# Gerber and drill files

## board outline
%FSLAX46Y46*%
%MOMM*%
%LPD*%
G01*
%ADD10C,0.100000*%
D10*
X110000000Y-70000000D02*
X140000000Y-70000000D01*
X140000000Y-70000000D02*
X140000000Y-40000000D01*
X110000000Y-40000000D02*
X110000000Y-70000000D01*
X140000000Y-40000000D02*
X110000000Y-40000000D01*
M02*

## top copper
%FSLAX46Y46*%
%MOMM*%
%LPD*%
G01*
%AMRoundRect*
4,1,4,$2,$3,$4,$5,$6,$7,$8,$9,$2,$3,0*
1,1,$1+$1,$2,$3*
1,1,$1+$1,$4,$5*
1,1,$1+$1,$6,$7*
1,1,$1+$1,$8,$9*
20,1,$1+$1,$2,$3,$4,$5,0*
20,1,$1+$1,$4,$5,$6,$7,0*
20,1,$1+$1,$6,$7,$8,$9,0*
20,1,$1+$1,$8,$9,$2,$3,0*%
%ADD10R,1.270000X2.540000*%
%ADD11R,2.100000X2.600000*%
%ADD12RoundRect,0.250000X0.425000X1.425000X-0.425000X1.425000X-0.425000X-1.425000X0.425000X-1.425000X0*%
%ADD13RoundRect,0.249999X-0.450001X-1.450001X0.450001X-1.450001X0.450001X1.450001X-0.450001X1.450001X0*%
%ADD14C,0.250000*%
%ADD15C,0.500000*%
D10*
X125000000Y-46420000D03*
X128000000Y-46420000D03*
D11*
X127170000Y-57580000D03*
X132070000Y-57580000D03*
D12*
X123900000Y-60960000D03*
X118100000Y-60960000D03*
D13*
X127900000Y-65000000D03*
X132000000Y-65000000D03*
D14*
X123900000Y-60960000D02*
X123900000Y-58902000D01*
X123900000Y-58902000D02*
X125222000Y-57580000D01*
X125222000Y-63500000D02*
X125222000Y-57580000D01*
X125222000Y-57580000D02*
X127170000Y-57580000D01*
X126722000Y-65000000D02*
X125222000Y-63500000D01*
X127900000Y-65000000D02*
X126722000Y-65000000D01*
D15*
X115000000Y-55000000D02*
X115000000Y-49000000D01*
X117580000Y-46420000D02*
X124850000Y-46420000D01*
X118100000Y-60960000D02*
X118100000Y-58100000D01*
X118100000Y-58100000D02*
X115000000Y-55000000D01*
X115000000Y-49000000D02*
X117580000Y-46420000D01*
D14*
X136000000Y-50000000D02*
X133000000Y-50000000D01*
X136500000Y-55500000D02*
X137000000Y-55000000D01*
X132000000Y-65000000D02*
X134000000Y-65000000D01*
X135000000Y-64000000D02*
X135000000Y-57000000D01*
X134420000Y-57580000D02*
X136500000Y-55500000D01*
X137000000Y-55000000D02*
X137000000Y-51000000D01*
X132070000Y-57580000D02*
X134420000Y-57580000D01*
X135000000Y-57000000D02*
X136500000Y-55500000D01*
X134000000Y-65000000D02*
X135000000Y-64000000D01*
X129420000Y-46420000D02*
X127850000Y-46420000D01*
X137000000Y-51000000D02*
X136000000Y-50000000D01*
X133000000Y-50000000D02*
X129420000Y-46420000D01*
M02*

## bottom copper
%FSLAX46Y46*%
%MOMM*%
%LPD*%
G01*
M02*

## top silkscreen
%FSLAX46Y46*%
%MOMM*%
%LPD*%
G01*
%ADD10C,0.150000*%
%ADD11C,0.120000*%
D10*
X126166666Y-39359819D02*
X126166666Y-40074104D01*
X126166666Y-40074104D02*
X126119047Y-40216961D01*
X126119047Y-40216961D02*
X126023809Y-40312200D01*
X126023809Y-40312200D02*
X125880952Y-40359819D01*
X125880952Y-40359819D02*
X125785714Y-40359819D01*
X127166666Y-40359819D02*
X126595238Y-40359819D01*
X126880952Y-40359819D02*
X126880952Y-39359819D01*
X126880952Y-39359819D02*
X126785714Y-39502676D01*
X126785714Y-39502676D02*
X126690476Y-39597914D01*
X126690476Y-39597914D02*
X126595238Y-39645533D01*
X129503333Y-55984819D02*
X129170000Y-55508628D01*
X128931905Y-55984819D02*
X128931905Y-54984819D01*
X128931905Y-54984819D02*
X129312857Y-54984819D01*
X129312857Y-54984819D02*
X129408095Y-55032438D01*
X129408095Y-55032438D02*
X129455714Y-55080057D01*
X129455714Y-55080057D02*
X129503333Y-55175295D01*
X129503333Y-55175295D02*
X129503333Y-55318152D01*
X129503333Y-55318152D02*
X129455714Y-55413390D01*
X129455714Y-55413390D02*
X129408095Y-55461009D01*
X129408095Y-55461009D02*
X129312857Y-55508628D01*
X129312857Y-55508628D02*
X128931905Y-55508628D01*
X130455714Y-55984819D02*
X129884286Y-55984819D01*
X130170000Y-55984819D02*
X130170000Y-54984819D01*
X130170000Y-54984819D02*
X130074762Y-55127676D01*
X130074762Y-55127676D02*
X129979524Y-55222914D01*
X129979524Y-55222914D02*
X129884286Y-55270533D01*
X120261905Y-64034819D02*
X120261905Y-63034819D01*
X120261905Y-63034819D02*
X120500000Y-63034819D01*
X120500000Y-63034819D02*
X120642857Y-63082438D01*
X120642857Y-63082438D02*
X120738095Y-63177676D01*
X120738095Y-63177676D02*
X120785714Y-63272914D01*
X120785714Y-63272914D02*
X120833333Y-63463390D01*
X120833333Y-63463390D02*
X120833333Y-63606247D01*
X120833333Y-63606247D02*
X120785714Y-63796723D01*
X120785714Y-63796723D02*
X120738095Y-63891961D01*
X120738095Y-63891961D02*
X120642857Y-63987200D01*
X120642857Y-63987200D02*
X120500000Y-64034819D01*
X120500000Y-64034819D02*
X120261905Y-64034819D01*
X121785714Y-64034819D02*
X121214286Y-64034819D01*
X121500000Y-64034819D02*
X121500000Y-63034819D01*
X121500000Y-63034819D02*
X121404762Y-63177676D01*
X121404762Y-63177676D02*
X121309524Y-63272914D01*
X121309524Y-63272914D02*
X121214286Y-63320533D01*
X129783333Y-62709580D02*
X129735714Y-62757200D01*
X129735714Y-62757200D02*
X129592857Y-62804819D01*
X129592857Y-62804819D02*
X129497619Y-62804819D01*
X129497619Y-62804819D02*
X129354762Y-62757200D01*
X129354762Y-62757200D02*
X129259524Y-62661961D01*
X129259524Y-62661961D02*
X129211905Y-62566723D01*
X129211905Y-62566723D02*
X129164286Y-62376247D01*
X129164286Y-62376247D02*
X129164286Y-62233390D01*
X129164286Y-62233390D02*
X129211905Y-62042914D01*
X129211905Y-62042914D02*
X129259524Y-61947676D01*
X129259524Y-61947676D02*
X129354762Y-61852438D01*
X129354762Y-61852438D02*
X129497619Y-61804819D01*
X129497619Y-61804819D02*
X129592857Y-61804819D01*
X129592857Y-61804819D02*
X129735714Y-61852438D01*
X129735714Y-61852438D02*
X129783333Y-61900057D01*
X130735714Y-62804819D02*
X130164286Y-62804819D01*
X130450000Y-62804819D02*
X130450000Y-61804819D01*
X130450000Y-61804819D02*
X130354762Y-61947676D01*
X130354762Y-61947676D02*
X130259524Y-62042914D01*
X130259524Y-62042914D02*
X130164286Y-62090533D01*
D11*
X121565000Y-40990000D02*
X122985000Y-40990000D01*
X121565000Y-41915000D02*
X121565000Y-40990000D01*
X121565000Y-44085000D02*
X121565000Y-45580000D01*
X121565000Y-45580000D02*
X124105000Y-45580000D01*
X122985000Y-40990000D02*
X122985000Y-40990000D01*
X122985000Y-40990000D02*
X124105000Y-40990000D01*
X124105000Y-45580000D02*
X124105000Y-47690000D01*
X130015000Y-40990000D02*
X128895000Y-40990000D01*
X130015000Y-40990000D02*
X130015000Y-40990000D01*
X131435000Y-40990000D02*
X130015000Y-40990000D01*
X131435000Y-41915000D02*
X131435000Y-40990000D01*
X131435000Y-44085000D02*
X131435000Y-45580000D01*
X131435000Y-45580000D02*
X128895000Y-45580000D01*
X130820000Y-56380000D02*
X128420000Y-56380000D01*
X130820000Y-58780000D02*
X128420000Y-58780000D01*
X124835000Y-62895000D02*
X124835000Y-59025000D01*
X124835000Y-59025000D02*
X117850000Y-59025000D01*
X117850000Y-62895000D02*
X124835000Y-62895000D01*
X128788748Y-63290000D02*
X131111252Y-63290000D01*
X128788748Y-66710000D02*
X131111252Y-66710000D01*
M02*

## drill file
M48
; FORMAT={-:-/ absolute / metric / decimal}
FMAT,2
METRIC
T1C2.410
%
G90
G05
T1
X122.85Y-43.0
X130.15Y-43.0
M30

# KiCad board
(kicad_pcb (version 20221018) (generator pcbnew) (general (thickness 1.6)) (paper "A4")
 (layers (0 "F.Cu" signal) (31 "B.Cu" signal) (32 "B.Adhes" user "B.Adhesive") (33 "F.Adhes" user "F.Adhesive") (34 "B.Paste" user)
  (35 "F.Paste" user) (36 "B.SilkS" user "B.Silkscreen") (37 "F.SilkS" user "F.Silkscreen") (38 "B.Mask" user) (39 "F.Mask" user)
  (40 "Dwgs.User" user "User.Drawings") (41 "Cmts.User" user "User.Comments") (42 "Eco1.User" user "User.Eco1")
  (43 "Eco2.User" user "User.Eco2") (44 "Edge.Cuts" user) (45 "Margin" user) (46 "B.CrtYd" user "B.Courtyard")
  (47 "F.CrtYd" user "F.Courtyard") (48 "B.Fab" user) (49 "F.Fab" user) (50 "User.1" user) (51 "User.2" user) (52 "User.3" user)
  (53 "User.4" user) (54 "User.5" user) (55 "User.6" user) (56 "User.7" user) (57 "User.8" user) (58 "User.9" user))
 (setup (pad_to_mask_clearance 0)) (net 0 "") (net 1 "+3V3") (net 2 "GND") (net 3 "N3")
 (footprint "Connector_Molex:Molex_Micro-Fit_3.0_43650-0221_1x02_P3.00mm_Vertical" (layer "F.Cu") (at 126.5 43.285)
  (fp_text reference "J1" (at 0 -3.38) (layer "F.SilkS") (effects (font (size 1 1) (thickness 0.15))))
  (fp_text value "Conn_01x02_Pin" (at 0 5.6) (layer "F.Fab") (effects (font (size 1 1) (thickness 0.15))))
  (fp_line (start -4.935 -2.295) (end -3.515 -2.295) (stroke (width 0.12) (type solid)) (layer "F.SilkS"))
  (fp_line (start -4.935 -1.37) (end -4.935 -2.295) (stroke (width 0.12) (type solid)) (layer "F.SilkS"))
  (fp_line (start -4.935 0.8) (end -4.935 2.295) (stroke (width 0.12) (type solid)) (layer "F.SilkS"))
  (fp_line (start -4.935 2.295) (end -2.395 2.295) (stroke (width 0.12) (type solid)) (layer "F.SilkS"))
  (fp_line (start -3.515 -2.295) (end -3.515 -2.295) (stroke (width 0.12) (type solid)) (layer "F.SilkS"))
  (fp_line (start -3.515 -2.295) (end -2.395 -2.295) (stroke (width 0.12) (type solid)) (layer "F.SilkS"))
  (fp_line (start -2.395 2.295) (end -2.395 4.405) (stroke (width 0.12) (type solid)) (layer "F.SilkS"))
  (fp_line (start 3.515 -2.295) (end 2.395 -2.295) (stroke (width 0.12) (type solid)) (layer "F.SilkS"))
  (fp_line (start 3.515 -2.295) (end 3.515 -2.295) (stroke (width 0.12) (type solid)) (layer "F.SilkS"))
  (fp_line (start 4.935 -2.295) (end 3.515 -2.295) (stroke (width 0.12) (type solid)) (layer "F.SilkS"))
  (fp_line (start 4.935 -1.37) (end 4.935 -2.295) (stroke (width 0.12) (type solid)) (layer "F.SilkS"))
  (fp_line (start 4.935 0.8) (end 4.935 2.295) (stroke (width 0.12) (type solid)) (layer "F.SilkS"))
  (fp_line (start 4.935 2.295) (end 2.395 2.295) (stroke (width 0.12) (type solid)) (layer "F.SilkS"))
  (pad "" np_thru_hole circle (at -3.65 -0.285) (size 2.41 2.41) (drill 2.41) (layers "*.Cu" "*.Mask"))
  (pad "" np_thru_hole circle (at 3.65 -0.285) (size 2.41 2.41) (drill 2.41) (layers "*.Cu" "*.Mask"))
  (pad "1" smd rect (at -1.5 3.135) (size 1.27 2.54) (layers "F.Cu" "F.Paste" "F.Mask") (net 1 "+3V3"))
  (pad "2" smd rect (at 1.5 3.135) (size 1.27 2.54) (layers "F.Cu" "F.Paste" "F.Mask") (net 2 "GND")))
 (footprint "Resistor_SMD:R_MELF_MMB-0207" (layer "F.Cu") (at 129.62 57.58)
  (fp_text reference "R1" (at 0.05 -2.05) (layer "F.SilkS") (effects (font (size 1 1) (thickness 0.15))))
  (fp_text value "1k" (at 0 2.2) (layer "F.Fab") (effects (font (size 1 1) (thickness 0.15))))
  (fp_line (start 1.2 -1.2) (end -1.2 -1.2) (stroke (width 0.12) (type solid)) (layer "F.SilkS"))
  (fp_line (start 1.2 1.2) (end -1.2 1.2) (stroke (width 0.12) (type solid)) (layer "F.SilkS"))
  (pad "1" smd rect (at -2.45 0) (size 2.1 2.6) (layers "F.Cu" "F.Paste" "F.Mask") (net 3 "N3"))
  (pad "2" smd rect (at 2.45 0) (size 2.1 2.6) (layers "F.Cu" "F.Paste" "F.Mask") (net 2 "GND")))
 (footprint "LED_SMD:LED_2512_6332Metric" (layer "F.Cu") (at 121 60.96 180)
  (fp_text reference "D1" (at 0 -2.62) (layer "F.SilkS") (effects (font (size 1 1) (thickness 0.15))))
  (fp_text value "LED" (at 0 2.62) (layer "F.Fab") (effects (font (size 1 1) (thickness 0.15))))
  (fp_line (start -3.835 -1.935) (end -3.835 1.935) (stroke (width 0.12) (type solid)) (layer "F.SilkS"))
  (fp_line (start -3.835 1.935) (end 3.15 1.935) (stroke (width 0.12) (type solid)) (layer "F.SilkS"))
  (fp_line (start 3.15 -1.935) (end -3.835 -1.935) (stroke (width 0.12) (type solid)) (layer "F.SilkS"))
  (pad "1" smd roundrect (at -2.9 0 180) (size 1.35 3.35) (layers "F.Cu" "F.Paste" "F.Mask") (roundrect_rratio 0.185185) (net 3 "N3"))
  (pad "2" smd roundrect (at 2.9 0 180) (size 1.35 3.35) (layers "F.Cu" "F.Paste" "F.Mask") (roundrect_rratio 0.185185) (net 1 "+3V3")))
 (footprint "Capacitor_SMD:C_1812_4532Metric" (layer "F.Cu") (at 129.95 65)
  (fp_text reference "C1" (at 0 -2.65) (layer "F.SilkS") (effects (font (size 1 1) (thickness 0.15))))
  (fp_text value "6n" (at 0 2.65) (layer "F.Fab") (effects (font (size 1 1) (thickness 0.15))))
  (fp_line (start -1.161252 -1.71) (end 1.161252 -1.71) (stroke (width 0.12) (type solid)) (layer "F.SilkS"))
  (fp_line (start -1.161252 1.71) (end 1.161252 1.71) (stroke (width 0.12) (type solid)) (layer "F.SilkS"))
  (pad "1" smd roundrect (at -2.05 0) (size 1.4 3.4) (layers "F.Cu" "F.Paste" "F.Mask") (roundrect_rratio 0.178571) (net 3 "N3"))
  (pad "2" smd roundrect (at 2.05 0) (size 1.4 3.4) (layers "F.Cu" "F.Paste" "F.Mask") (roundrect_rratio 0.178571) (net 2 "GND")))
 (gr_line (start 110 70) (end 140 70) (stroke (width 0.1) (type default)) (layer "Edge.Cuts"))
 (gr_line (start 140 70) (end 140 40) (stroke (width 0.1) (type default)) (layer "Edge.Cuts"))
 (gr_line (start 110 40) (end 110 70) (stroke (width 0.1) (type default)) (layer "Edge.Cuts"))
 (gr_line (start 140 40) (end 110 40) (stroke (width 0.1) (type default)) (layer "Edge.Cuts"))
 (segment (start 123.9 60.96) (end 123.9 58.902) (width 0.25) (layer "F.Cu") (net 3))
 (segment (start 123.9 58.902) (end 125.222 57.58) (width 0.25) (layer "F.Cu") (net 3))
 (segment (start 125.222 63.5) (end 125.222 57.58) (width 0.25) (layer "F.Cu") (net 3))
 (segment (start 125.222 57.58) (end 127.17 57.58) (width 0.25) (layer "F.Cu") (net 3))
 (segment (start 126.722 65) (end 125.222 63.5) (width 0.25) (layer "F.Cu") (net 3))
 (segment (start 127.9 65) (end 126.722 65) (width 0.25) (layer "F.Cu") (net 3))
 (segment (start 115 55) (end 115 49) (width 0.5) (layer "F.Cu") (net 1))
 (segment (start 117.58 46.42) (end 124.85 46.42) (width 0.5) (layer "F.Cu") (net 1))
 (segment (start 118.1 60.96) (end 118.1 58.1) (width 0.5) (layer "F.Cu") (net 1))
 (segment (start 118.1 58.1) (end 115 55) (width 0.5) (layer "F.Cu") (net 1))
 (segment (start 115 49) (end 117.58 46.42) (width 0.5) (layer "F.Cu") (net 1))
 (segment (start 136 50) (end 133 50) (width 0.25) (layer "F.Cu") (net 2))
 (segment (start 136.5 55.5) (end 137 55) (width 0.25) (layer "F.Cu") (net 2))
 (segment (start 132 65) (end 134 65) (width 0.25) (layer "F.Cu") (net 2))
 (segment (start 135 64) (end 135 57) (width 0.25) (layer "F.Cu") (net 2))
 (segment (start 134.42 57.58) (end 136.5 55.5) (width 0.25) (layer "F.Cu") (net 2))
 (segment (start 137 55) (end 137 51) (width 0.25) (layer "F.Cu") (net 2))
 (segment (start 132.07 57.58) (end 134.42 57.58) (width 0.25) (layer "F.Cu") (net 2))
 (segment (start 135 57) (end 136.5 55.5) (width 0.25) (layer "F.Cu") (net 2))
 (segment (start 134 65) (end 135 64) (width 0.25) (layer "F.Cu") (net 2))
 (segment (start 129.42 46.42) (end 127.85 46.42) (width 0.25) (layer "F.Cu") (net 2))
 (segment (start 137 51) (end 136 50) (width 0.25) (layer "F.Cu") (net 2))
 (segment (start 133 50) (end 129.42 46.42) (width 0.25) (layer "F.Cu") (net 2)))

